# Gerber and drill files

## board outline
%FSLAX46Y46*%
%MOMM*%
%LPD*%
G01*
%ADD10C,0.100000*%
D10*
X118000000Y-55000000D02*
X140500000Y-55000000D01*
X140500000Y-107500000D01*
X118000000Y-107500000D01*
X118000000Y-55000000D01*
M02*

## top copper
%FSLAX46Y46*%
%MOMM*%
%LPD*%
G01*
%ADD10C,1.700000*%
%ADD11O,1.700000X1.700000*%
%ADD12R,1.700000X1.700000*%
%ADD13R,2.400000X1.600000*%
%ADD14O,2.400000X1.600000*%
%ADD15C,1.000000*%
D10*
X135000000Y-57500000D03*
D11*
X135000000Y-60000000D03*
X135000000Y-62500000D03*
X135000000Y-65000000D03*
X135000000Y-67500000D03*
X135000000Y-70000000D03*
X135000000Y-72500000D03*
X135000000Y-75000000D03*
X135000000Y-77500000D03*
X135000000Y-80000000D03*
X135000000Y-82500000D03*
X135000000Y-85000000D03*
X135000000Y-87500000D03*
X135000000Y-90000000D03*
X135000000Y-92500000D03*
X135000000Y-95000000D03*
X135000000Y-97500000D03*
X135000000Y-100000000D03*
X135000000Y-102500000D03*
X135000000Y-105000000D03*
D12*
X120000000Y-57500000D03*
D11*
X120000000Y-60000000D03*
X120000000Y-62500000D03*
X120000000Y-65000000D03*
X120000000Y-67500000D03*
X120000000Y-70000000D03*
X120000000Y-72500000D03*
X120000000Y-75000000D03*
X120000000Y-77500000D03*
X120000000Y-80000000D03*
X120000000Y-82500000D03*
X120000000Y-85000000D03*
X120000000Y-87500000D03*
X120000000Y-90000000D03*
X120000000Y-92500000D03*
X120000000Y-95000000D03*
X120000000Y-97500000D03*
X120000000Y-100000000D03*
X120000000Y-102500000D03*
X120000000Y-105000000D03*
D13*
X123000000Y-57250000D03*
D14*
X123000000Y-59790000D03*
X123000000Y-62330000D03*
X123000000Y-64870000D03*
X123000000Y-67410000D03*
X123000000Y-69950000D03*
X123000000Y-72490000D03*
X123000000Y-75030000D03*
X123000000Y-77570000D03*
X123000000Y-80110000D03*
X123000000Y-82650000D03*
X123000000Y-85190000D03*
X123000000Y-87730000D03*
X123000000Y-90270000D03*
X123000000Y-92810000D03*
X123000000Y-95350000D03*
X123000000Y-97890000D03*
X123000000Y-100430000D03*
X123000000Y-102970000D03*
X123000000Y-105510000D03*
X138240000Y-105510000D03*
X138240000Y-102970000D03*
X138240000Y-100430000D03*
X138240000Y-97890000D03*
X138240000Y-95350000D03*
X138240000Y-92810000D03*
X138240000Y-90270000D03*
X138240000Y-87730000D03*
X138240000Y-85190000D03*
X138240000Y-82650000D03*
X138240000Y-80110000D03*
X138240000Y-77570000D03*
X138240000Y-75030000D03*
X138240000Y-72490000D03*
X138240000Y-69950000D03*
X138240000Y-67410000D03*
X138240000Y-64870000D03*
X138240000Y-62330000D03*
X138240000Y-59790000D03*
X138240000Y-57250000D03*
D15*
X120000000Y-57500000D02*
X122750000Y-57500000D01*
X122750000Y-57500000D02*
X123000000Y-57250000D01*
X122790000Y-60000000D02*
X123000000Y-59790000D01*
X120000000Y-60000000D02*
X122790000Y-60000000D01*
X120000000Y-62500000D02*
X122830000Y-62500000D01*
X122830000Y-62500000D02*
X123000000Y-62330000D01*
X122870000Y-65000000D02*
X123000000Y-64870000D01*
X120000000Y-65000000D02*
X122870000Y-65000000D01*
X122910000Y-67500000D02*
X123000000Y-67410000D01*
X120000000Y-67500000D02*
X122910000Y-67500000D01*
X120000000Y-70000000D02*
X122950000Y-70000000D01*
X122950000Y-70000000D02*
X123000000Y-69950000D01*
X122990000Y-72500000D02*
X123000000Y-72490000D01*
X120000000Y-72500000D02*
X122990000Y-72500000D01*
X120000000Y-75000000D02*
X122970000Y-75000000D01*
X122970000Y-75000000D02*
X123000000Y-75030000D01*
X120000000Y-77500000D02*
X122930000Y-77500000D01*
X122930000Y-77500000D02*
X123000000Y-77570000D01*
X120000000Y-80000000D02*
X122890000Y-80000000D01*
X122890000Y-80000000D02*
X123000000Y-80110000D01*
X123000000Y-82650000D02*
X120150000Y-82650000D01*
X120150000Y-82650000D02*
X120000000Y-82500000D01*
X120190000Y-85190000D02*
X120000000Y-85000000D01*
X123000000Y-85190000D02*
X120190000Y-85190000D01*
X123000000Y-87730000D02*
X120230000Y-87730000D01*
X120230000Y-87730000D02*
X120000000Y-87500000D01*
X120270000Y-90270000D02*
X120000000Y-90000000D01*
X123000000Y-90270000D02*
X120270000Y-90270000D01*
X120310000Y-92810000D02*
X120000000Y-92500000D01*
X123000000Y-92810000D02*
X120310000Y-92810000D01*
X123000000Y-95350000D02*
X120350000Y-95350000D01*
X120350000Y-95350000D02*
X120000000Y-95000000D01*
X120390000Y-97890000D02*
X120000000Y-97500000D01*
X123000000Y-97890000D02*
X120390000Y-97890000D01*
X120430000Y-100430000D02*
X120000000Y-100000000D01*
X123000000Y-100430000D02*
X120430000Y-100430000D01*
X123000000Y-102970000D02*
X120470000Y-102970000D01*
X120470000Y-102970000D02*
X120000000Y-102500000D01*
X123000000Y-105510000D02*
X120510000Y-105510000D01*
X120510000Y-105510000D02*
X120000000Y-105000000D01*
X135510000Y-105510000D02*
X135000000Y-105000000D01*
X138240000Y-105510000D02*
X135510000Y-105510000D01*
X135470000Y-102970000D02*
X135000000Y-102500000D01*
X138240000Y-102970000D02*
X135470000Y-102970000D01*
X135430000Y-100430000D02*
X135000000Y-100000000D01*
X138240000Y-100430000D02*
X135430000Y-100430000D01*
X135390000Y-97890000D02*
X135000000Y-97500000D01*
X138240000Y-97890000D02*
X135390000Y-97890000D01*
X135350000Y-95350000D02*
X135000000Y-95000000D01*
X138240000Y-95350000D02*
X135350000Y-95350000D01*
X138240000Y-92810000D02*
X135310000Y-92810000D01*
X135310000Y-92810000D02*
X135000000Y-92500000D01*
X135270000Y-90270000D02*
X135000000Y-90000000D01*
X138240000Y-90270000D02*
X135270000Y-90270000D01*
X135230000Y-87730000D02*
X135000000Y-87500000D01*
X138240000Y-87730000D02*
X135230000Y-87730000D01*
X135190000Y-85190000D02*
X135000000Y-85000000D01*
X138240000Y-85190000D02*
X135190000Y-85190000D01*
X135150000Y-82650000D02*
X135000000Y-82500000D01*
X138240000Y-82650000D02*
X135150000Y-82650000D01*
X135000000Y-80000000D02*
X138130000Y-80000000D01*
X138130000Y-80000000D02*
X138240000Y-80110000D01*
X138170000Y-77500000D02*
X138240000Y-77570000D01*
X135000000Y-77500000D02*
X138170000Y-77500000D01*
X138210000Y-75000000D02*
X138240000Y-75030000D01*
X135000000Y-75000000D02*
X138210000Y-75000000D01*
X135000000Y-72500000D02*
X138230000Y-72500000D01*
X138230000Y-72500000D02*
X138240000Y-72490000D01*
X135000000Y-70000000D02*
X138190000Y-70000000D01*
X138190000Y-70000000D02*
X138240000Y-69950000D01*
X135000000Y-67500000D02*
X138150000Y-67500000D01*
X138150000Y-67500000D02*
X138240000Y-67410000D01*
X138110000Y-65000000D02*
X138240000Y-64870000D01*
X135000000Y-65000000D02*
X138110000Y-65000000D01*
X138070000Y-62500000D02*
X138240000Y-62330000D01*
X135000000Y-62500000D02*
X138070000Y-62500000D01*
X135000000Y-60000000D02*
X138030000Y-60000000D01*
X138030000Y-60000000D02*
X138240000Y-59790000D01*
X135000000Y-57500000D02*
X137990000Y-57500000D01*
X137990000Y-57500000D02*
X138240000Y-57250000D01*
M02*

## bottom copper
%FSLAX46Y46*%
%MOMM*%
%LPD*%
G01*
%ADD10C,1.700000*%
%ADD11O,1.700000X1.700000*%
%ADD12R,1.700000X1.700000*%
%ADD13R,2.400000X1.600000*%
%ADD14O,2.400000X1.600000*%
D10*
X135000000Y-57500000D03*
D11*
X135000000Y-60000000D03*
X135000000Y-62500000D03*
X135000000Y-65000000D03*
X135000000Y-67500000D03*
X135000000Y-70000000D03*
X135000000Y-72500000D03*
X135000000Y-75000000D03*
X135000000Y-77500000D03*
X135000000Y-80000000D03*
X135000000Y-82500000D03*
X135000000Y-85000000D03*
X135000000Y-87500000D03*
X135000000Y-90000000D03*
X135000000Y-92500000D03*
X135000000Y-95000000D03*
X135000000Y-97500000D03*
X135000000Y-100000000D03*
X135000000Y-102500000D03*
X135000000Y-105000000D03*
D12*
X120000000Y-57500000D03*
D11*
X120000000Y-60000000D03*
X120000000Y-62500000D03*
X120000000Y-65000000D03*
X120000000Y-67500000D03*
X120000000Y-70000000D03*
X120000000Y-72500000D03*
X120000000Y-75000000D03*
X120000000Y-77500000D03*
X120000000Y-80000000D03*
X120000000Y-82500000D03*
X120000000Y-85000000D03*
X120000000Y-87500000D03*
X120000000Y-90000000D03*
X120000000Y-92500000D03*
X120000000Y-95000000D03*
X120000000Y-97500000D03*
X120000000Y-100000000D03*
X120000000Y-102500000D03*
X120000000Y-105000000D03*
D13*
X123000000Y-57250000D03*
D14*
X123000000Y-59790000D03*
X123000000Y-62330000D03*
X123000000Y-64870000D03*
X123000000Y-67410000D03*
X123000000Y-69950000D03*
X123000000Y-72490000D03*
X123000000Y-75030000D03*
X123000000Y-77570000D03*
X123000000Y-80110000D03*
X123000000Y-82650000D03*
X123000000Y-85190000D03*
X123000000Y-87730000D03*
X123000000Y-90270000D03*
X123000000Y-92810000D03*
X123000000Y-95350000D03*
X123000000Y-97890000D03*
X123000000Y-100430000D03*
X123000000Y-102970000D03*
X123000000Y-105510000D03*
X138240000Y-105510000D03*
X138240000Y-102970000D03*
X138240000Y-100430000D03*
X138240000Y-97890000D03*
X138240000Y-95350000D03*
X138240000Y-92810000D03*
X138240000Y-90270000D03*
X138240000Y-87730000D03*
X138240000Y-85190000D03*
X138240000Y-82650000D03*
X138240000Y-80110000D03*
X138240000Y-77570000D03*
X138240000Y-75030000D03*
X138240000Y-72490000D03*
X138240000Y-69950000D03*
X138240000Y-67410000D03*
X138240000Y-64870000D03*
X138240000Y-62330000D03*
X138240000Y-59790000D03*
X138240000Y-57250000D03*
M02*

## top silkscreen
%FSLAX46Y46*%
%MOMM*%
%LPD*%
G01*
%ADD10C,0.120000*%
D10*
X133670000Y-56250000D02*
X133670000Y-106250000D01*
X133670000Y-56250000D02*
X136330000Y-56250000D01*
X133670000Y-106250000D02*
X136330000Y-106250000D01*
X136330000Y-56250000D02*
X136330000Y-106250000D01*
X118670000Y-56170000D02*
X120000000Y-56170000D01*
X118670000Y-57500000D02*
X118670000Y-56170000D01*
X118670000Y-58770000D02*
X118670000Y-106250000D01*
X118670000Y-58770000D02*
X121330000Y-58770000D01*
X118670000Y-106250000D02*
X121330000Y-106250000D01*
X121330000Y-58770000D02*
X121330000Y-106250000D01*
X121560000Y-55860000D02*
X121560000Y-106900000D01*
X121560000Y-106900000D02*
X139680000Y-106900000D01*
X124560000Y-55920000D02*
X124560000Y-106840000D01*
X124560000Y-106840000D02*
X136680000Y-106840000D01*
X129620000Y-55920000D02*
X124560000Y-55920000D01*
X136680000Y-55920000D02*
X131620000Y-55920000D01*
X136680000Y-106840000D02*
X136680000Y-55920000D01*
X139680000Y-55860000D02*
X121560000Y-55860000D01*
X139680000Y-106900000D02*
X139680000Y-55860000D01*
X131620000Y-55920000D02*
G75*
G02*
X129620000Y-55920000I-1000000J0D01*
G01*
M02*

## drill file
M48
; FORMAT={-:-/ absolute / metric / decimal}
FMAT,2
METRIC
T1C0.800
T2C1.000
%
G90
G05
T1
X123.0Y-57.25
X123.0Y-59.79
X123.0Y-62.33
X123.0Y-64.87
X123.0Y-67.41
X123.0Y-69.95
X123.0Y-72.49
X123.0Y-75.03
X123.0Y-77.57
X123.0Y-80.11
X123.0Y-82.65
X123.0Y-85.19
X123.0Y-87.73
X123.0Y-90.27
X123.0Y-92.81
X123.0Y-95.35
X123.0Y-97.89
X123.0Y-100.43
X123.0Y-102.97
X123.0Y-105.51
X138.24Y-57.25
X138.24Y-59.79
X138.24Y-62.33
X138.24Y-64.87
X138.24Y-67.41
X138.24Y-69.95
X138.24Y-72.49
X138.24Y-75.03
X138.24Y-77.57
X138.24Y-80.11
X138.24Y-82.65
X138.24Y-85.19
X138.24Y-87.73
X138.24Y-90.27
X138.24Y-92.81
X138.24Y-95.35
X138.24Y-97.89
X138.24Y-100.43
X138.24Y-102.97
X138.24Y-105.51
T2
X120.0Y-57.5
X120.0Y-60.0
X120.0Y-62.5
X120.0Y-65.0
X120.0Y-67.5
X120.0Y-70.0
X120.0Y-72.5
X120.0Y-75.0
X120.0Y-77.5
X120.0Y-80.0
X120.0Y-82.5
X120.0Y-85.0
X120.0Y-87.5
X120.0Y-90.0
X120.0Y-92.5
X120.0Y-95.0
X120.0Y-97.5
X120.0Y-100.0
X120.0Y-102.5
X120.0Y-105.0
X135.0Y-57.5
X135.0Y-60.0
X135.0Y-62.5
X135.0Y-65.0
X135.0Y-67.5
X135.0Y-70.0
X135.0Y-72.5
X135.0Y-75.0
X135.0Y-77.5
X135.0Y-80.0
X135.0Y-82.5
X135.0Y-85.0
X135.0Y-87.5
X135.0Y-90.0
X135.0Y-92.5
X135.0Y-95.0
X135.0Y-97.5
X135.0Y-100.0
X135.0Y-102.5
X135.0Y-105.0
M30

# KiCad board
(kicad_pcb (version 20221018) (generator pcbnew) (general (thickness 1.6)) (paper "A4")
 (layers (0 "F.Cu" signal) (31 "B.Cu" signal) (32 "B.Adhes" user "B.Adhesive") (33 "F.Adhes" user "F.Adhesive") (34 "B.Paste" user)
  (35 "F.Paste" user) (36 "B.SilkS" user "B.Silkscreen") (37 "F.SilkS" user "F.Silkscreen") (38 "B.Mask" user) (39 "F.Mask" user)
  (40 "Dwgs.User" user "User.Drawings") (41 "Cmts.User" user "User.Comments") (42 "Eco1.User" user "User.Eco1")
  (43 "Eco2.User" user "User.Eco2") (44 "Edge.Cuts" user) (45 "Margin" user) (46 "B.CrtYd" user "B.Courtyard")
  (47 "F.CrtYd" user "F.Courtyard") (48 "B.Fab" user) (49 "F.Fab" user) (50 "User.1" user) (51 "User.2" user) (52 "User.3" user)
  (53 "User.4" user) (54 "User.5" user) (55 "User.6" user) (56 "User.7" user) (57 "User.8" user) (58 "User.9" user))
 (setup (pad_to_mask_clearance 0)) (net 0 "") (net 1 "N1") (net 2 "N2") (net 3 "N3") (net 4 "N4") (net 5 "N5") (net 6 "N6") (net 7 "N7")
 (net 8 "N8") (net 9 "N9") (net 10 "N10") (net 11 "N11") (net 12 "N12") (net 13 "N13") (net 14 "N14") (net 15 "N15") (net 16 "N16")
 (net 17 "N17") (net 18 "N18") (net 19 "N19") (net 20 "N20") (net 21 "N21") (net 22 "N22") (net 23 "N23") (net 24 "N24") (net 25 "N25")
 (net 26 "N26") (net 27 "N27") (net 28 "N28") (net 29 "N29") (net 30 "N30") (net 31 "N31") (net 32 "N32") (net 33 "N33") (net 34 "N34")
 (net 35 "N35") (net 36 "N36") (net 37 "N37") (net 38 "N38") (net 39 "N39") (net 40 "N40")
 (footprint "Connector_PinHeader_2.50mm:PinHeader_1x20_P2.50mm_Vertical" (layer "F.Cu") (at 135 60)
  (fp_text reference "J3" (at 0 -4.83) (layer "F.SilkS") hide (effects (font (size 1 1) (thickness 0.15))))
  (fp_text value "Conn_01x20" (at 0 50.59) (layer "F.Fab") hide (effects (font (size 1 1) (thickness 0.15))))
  (fp_line (start -1.33 -3.75) (end -1.33 46.25) (stroke (width 0.12) (type solid)) (layer "F.SilkS"))
  (fp_line (start -1.33 -3.75) (end 1.33 -3.75) (stroke (width 0.12) (type solid)) (layer "F.SilkS"))
  (fp_line (start -1.33 46.25) (end 1.33 46.25) (stroke (width 0.12) (type solid)) (layer "F.SilkS"))
  (fp_line (start 1.33 -3.75) (end 1.33 46.25) (stroke (width 0.12) (type solid)) (layer "F.SilkS"))
  (pad "1" thru_hole circle (at 0 -2.5) (size 1.7 1.7) (drill 1) (layers "*.Cu" "*.Mask") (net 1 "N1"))
  (pad "2" thru_hole oval (at 0 0) (size 1.7 1.7) (drill 1) (layers "*.Cu" "*.Mask") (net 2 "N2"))
  (pad "3" thru_hole oval (at 0 2.5) (size 1.7 1.7) (drill 1) (layers "*.Cu" "*.Mask") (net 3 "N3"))
  (pad "4" thru_hole oval (at 0 5) (size 1.7 1.7) (drill 1) (layers "*.Cu" "*.Mask") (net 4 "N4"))
  (pad "5" thru_hole oval (at 0 7.5) (size 1.7 1.7) (drill 1) (layers "*.Cu" "*.Mask") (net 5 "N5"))
  (pad "6" thru_hole oval (at 0 10) (size 1.7 1.7) (drill 1) (layers "*.Cu" "*.Mask") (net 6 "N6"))
  (pad "7" thru_hole oval (at 0 12.5) (size 1.7 1.7) (drill 1) (layers "*.Cu" "*.Mask") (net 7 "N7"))
  (pad "8" thru_hole oval (at 0 15) (size 1.7 1.7) (drill 1) (layers "*.Cu" "*.Mask") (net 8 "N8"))
  (pad "9" thru_hole oval (at 0 17.5) (size 1.7 1.7) (drill 1) (layers "*.Cu" "*.Mask") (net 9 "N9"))
  (pad "10" thru_hole oval (at 0 20) (size 1.7 1.7) (drill 1) (layers "*.Cu" "*.Mask") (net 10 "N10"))
  (pad "11" thru_hole oval (at 0 22.5) (size 1.7 1.7) (drill 1) (layers "*.Cu" "*.Mask") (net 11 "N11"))
  (pad "12" thru_hole oval (at 0 25) (size 1.7 1.7) (drill 1) (layers "*.Cu" "*.Mask") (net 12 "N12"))
  (pad "13" thru_hole oval (at 0 27.5) (size 1.7 1.7) (drill 1) (layers "*.Cu" "*.Mask") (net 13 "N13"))
  (pad "14" thru_hole oval (at 0 30) (size 1.7 1.7) (drill 1) (layers "*.Cu" "*.Mask") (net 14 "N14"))
  (pad "15" thru_hole oval (at 0 32.5) (size 1.7 1.7) (drill 1) (layers "*.Cu" "*.Mask") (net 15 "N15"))
  (pad "16" thru_hole oval (at 0 35) (size 1.7 1.7) (drill 1) (layers "*.Cu" "*.Mask") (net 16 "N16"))
  (pad "17" thru_hole oval (at 0 37.5) (size 1.7 1.7) (drill 1) (layers "*.Cu" "*.Mask") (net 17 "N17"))
  (pad "18" thru_hole oval (at 0 40) (size 1.7 1.7) (drill 1) (layers "*.Cu" "*.Mask") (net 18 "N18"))
  (pad "19" thru_hole oval (at 0 42.5) (size 1.7 1.7) (drill 1) (layers "*.Cu" "*.Mask") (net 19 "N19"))
  (pad "20" thru_hole oval (at 0 45) (size 1.7 1.7) (drill 1) (layers "*.Cu" "*.Mask") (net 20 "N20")))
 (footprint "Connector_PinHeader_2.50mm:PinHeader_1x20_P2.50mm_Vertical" (layer "F.Cu") (at 120 60)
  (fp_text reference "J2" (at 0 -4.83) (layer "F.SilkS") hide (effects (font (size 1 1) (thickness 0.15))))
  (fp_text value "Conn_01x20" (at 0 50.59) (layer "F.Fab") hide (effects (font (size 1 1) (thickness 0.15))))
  (fp_line (start -1.33 -3.83) (end 0 -3.83) (stroke (width 0.12) (type solid)) (layer "F.SilkS"))
  (fp_line (start -1.33 -2.5) (end -1.33 -3.83) (stroke (width 0.12) (type solid)) (layer "F.SilkS"))
  (fp_line (start -1.33 -1.23) (end -1.33 46.25) (stroke (width 0.12) (type solid)) (layer "F.SilkS"))
  (fp_line (start -1.33 -1.23) (end 1.33 -1.23) (stroke (width 0.12) (type solid)) (layer "F.SilkS"))
  (fp_line (start -1.33 46.25) (end 1.33 46.25) (stroke (width 0.12) (type solid)) (layer "F.SilkS"))
  (fp_line (start 1.33 -1.23) (end 1.33 46.25) (stroke (width 0.12) (type solid)) (layer "F.SilkS"))
  (pad "1" thru_hole rect (at 0 -2.5) (size 1.7 1.7) (drill 1) (layers "*.Cu" "*.Mask") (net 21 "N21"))
  (pad "2" thru_hole oval (at 0 0) (size 1.7 1.7) (drill 1) (layers "*.Cu" "*.Mask") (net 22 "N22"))
  (pad "3" thru_hole oval (at 0 2.5) (size 1.7 1.7) (drill 1) (layers "*.Cu" "*.Mask") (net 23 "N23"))
  (pad "4" thru_hole oval (at 0 5) (size 1.7 1.7) (drill 1) (layers "*.Cu" "*.Mask") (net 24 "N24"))
  (pad "5" thru_hole oval (at 0 7.5) (size 1.7 1.7) (drill 1) (layers "*.Cu" "*.Mask") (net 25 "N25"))
  (pad "6" thru_hole oval (at 0 10) (size 1.7 1.7) (drill 1) (layers "*.Cu" "*.Mask") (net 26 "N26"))
  (pad "7" thru_hole oval (at 0 12.5) (size 1.7 1.7) (drill 1) (layers "*.Cu" "*.Mask") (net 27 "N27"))
  (pad "8" thru_hole oval (at 0 15) (size 1.7 1.7) (drill 1) (layers "*.Cu" "*.Mask") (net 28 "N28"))
  (pad "9" thru_hole oval (at 0 17.5) (size 1.7 1.7) (drill 1) (layers "*.Cu" "*.Mask") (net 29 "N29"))
  (pad "10" thru_hole oval (at 0 20) (size 1.7 1.7) (drill 1) (layers "*.Cu" "*.Mask") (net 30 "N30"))
  (pad "11" thru_hole oval (at 0 22.5) (size 1.7 1.7) (drill 1) (layers "*.Cu" "*.Mask") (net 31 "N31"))
  (pad "12" thru_hole oval (at 0 25) (size 1.7 1.7) (drill 1) (layers "*.Cu" "*.Mask") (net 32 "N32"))
  (pad "13" thru_hole oval (at 0 27.5) (size 1.7 1.7) (drill 1) (layers "*.Cu" "*.Mask") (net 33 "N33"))
  (pad "14" thru_hole oval (at 0 30) (size 1.7 1.7) (drill 1) (layers "*.Cu" "*.Mask") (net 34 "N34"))
  (pad "15" thru_hole oval (at 0 32.5) (size 1.7 1.7) (drill 1) (layers "*.Cu" "*.Mask") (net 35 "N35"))
  (pad "16" thru_hole oval (at 0 35) (size 1.7 1.7) (drill 1) (layers "*.Cu" "*.Mask") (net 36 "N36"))
  (pad "17" thru_hole oval (at 0 37.5) (size 1.7 1.7) (drill 1) (layers "*.Cu" "*.Mask") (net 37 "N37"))
  (pad "18" thru_hole oval (at 0 40) (size 1.7 1.7) (drill 1) (layers "*.Cu" "*.Mask") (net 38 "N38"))
  (pad "19" thru_hole oval (at 0 42.5) (size 1.7 1.7) (drill 1) (layers "*.Cu" "*.Mask") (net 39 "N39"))
  (pad "20" thru_hole oval (at 0 45) (size 1.7 1.7) (drill 1) (layers "*.Cu" "*.Mask") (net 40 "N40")))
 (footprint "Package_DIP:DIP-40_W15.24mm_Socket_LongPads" (layer "F.Cu") (at 123 57.25)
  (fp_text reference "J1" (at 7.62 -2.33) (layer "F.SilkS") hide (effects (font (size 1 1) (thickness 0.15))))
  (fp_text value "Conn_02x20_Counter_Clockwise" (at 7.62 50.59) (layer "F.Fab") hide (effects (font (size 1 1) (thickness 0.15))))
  (fp_line (start -1.44 -1.39) (end -1.44 49.65) (stroke (width 0.12) (type solid)) (layer "F.SilkS"))
  (fp_line (start -1.44 49.65) (end 16.68 49.65) (stroke (width 0.12) (type solid)) (layer "F.SilkS"))
  (fp_line (start 1.56 -1.33) (end 1.56 49.59) (stroke (width 0.12) (type solid)) (layer "F.SilkS"))
  (fp_line (start 1.56 49.59) (end 13.68 49.59) (stroke (width 0.12) (type solid)) (layer "F.SilkS"))
  (fp_line (start 6.62 -1.33) (end 1.56 -1.33) (stroke (width 0.12) (type solid)) (layer "F.SilkS"))
  (fp_line (start 13.68 -1.33) (end 8.62 -1.33) (stroke (width 0.12) (type solid)) (layer "F.SilkS"))
  (fp_line (start 13.68 49.59) (end 13.68 -1.33) (stroke (width 0.12) (type solid)) (layer "F.SilkS"))
  (fp_line (start 16.68 -1.39) (end -1.44 -1.39) (stroke (width 0.12) (type solid)) (layer "F.SilkS"))
  (fp_line (start 16.68 49.65) (end 16.68 -1.39) (stroke (width 0.12) (type solid)) (layer "F.SilkS"))
  (fp_arc (start 8.62 -1.33) (mid 7.62 -0.33) (end 6.62 -1.33) (stroke (width 0.12) (type solid)) (layer "F.SilkS"))
  (pad "1" thru_hole rect (at 0 0) (size 2.4 1.6) (drill 0.8) (layers "*.Cu" "*.Mask") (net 21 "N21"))
  (pad "2" thru_hole oval (at 0 2.54) (size 2.4 1.6) (drill 0.8) (layers "*.Cu" "*.Mask") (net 22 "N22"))
  (pad "3" thru_hole oval (at 0 5.08) (size 2.4 1.6) (drill 0.8) (layers "*.Cu" "*.Mask") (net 23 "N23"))
  (pad "4" thru_hole oval (at 0 7.62) (size 2.4 1.6) (drill 0.8) (layers "*.Cu" "*.Mask") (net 24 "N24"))
  (pad "5" thru_hole oval (at 0 10.16) (size 2.4 1.6) (drill 0.8) (layers "*.Cu" "*.Mask") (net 25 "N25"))
  (pad "6" thru_hole oval (at 0 12.7) (size 2.4 1.6) (drill 0.8) (layers "*.Cu" "*.Mask") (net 26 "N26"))
  (pad "7" thru_hole oval (at 0 15.24) (size 2.4 1.6) (drill 0.8) (layers "*.Cu" "*.Mask") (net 27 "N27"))
  (pad "8" thru_hole oval (at 0 17.78) (size 2.4 1.6) (drill 0.8) (layers "*.Cu" "*.Mask") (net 28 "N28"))
  (pad "9" thru_hole oval (at 0 20.32) (size 2.4 1.6) (drill 0.8) (layers "*.Cu" "*.Mask") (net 29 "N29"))
  (pad "10" thru_hole oval (at 0 22.86) (size 2.4 1.6) (drill 0.8) (layers "*.Cu" "*.Mask") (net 30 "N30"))
  (pad "11" thru_hole oval (at 0 25.4) (size 2.4 1.6) (drill 0.8) (layers "*.Cu" "*.Mask") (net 31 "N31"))
  (pad "12" thru_hole oval (at 0 27.94) (size 2.4 1.6) (drill 0.8) (layers "*.Cu" "*.Mask") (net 32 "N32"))
  (pad "13" thru_hole oval (at 0 30.48) (size 2.4 1.6) (drill 0.8) (layers "*.Cu" "*.Mask") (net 33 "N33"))
  (pad "14" thru_hole oval (at 0 33.02) (size 2.4 1.6) (drill 0.8) (layers "*.Cu" "*.Mask") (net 34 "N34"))
  (pad "15" thru_hole oval (at 0 35.56) (size 2.4 1.6) (drill 0.8) (layers "*.Cu" "*.Mask") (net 35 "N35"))
  (pad "16" thru_hole oval (at 0 38.1) (size 2.4 1.6) (drill 0.8) (layers "*.Cu" "*.Mask") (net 36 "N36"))
  (pad "17" thru_hole oval (at 0 40.64) (size 2.4 1.6) (drill 0.8) (layers "*.Cu" "*.Mask") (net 37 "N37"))
  (pad "18" thru_hole oval (at 0 43.18) (size 2.4 1.6) (drill 0.8) (layers "*.Cu" "*.Mask") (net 38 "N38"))
  (pad "19" thru_hole oval (at 0 45.72) (size 2.4 1.6) (drill 0.8) (layers "*.Cu" "*.Mask") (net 39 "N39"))
  (pad "20" thru_hole oval (at 0 48.26) (size 2.4 1.6) (drill 0.8) (layers "*.Cu" "*.Mask") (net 40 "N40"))
  (pad "21" thru_hole oval (at 15.24 48.26) (size 2.4 1.6) (drill 0.8) (layers "*.Cu" "*.Mask") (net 20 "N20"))
  (pad "22" thru_hole oval (at 15.24 45.72) (size 2.4 1.6) (drill 0.8) (layers "*.Cu" "*.Mask") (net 19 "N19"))
  (pad "23" thru_hole oval (at 15.24 43.18) (size 2.4 1.6) (drill 0.8) (layers "*.Cu" "*.Mask") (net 18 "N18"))
  (pad "24" thru_hole oval (at 15.24 40.64) (size 2.4 1.6) (drill 0.8) (layers "*.Cu" "*.Mask") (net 17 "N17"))
  (pad "25" thru_hole oval (at 15.24 38.1) (size 2.4 1.6) (drill 0.8) (layers "*.Cu" "*.Mask") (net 16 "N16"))
  (pad "26" thru_hole oval (at 15.24 35.56) (size 2.4 1.6) (drill 0.8) (layers "*.Cu" "*.Mask") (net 15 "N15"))
  (pad "27" thru_hole oval (at 15.24 33.02) (size 2.4 1.6) (drill 0.8) (layers "*.Cu" "*.Mask") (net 14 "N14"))
  (pad "28" thru_hole oval (at 15.24 30.48) (size 2.4 1.6) (drill 0.8) (layers "*.Cu" "*.Mask") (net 13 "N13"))
  (pad "29" thru_hole oval (at 15.24 27.94) (size 2.4 1.6) (drill 0.8) (layers "*.Cu" "*.Mask") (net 12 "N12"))
  (pad "30" thru_hole oval (at 15.24 25.4) (size 2.4 1.6) (drill 0.8) (layers "*.Cu" "*.Mask") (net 11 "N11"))
  (pad "31" thru_hole oval (at 15.24 22.86) (size 2.4 1.6) (drill 0.8) (layers "*.Cu" "*.Mask") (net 10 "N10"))
  (pad "32" thru_hole oval (at 15.24 20.32) (size 2.4 1.6) (drill 0.8) (layers "*.Cu" "*.Mask") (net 9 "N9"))
  (pad "33" thru_hole oval (at 15.24 17.78) (size 2.4 1.6) (drill 0.8) (layers "*.Cu" "*.Mask") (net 8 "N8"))
  (pad "34" thru_hole oval (at 15.24 15.24) (size 2.4 1.6) (drill 0.8) (layers "*.Cu" "*.Mask") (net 7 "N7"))
  (pad "35" thru_hole oval (at 15.24 12.7) (size 2.4 1.6) (drill 0.8) (layers "*.Cu" "*.Mask") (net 6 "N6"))
  (pad "36" thru_hole oval (at 15.24 10.16) (size 2.4 1.6) (drill 0.8) (layers "*.Cu" "*.Mask") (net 5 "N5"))
  (pad "37" thru_hole oval (at 15.24 7.62) (size 2.4 1.6) (drill 0.8) (layers "*.Cu" "*.Mask") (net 4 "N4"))
  (pad "38" thru_hole oval (at 15.24 5.08) (size 2.4 1.6) (drill 0.8) (layers "*.Cu" "*.Mask") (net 3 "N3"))
  (pad "39" thru_hole oval (at 15.24 2.54) (size 2.4 1.6) (drill 0.8) (layers "*.Cu" "*.Mask") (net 2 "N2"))
  (pad "40" thru_hole oval (at 15.24 0) (size 2.4 1.6) (drill 0.8) (layers "*.Cu" "*.Mask") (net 1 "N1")))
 (gr_rect (start 118 55) (end 140.5 107.5) (stroke (width 0.1) (type default)) (fill none) (layer "Edge.Cuts"))
 (segment (start 120 57.5) (end 122.75 57.5) (width 1) (layer "F.Cu") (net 21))
 (segment (start 122.75 57.5) (end 123 57.25) (width 1) (layer "F.Cu") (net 21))
 (segment (start 122.79 60) (end 123 59.79) (width 1) (layer "F.Cu") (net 22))
 (segment (start 120 60) (end 122.79 60) (width 1) (layer "F.Cu") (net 22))
 (segment (start 120 62.5) (end 122.83 62.5) (width 1) (layer "F.Cu") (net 23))
 (segment (start 122.83 62.5) (end 123 62.33) (width 1) (layer "F.Cu") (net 23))
 (segment (start 122.87 65) (end 123 64.87) (width 1) (layer "F.Cu") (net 24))
 (segment (start 120 65) (end 122.87 65) (width 1) (layer "F.Cu") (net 24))
 (segment (start 122.91 67.5) (end 123 67.41) (width 1) (layer "F.Cu") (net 25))
 (segment (start 120 67.5) (end 122.91 67.5) (width 1) (layer "F.Cu") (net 25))
 (segment (start 120 70) (end 122.95 70) (width 1) (layer "F.Cu") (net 26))
 (segment (start 122.95 70) (end 123 69.95) (width 1) (layer "F.Cu") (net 26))
 (segment (start 122.99 72.5) (end 123 72.49) (width 1) (layer "F.Cu") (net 27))
 (segment (start 120 72.5) (end 122.99 72.5) (width 1) (layer "F.Cu") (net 27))
 (segment (start 120 75) (end 122.97 75) (width 1) (layer "F.Cu") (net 28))
 (segment (start 122.97 75) (end 123 75.03) (width 1) (layer "F.Cu") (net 28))
 (segment (start 120 77.5) (end 122.93 77.5) (width 1) (layer "F.Cu") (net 29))
 (segment (start 122.93 77.5) (end 123 77.57) (width 1) (layer "F.Cu") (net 29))
 (segment (start 120 80) (end 122.89 80) (width 1) (layer "F.Cu") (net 30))
 (segment (start 122.89 80) (end 123 80.11) (width 1) (layer "F.Cu") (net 30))
 (segment (start 123 82.65) (end 120.15 82.65) (width 1) (layer "F.Cu") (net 31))
 (segment (start 120.15 82.65) (end 120 82.5) (width 1) (layer "F.Cu") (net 31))
 (segment (start 120.19 85.19) (end 120 85) (width 1) (layer "F.Cu") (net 32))
 (segment (start 123 85.19) (end 120.19 85.19) (width 1) (layer "F.Cu") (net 32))
 (segment (start 123 87.73) (end 120.23 87.73) (width 1) (layer "F.Cu") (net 33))
 (segment (start 120.23 87.73) (end 120 87.5) (width 1) (layer "F.Cu") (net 33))
 (segment (start 120.27 90.27) (end 120 90) (width 1) (layer "F.Cu") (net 34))
 (segment (start 123 90.27) (end 120.27 90.27) (width 1) (layer "F.Cu") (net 34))
 (segment (start 120.31 92.81) (end 120 92.5) (width 1) (layer "F.Cu") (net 35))
 (segment (start 123 92.81) (end 120.31 92.81) (width 1) (layer "F.Cu") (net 35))
 (segment (start 123 95.35) (end 120.35 95.35) (width 1) (layer "F.Cu") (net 36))
 (segment (start 120.35 95.35) (end 120 95) (width 1) (layer "F.Cu") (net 36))
 (segment (start 120.39 97.89) (end 120 97.5) (width 1) (layer "F.Cu") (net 37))
 (segment (start 123 97.89) (end 120.39 97.89) (width 1) (layer "F.Cu") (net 37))
 (segment (start 120.43 100.43) (end 120 100) (width 1) (layer "F.Cu") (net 38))
 (segment (start 123 100.43) (end 120.43 100.43) (width 1) (layer "F.Cu") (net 38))
 (segment (start 123 102.97) (end 120.47 102.97) (width 1) (layer "F.Cu") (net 39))
 (segment (start 120.47 102.97) (end 120 102.5) (width 1) (layer "F.Cu") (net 39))
 (segment (start 123 105.51) (end 120.51 105.51) (width 1) (layer "F.Cu") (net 40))
 (segment (start 120.51 105.51) (end 120 105) (width 1) (layer "F.Cu") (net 40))
 (segment (start 135.51 105.51) (end 135 105) (width 1) (layer "F.Cu") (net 20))
 (segment (start 138.24 105.51) (end 135.51 105.51) (width 1) (layer "F.Cu") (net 20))
 (segment (start 135.47 102.97) (end 135 102.5) (width 1) (layer "F.Cu") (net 19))
 (segment (start 138.24 102.97) (end 135.47 102.97) (width 1) (layer "F.Cu") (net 19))
 (segment (start 135.43 100.43) (end 135 100) (width 1) (layer "F.Cu") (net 18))
 (segment (start 138.24 100.43) (end 135.43 100.43) (width 1) (layer "F.Cu") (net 18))
 (segment (start 135.39 97.89) (end 135 97.5) (width 1) (layer "F.Cu") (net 17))
 (segment (start 138.24 97.89) (end 135.39 97.89) (width 1) (layer "F.Cu") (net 17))
 (segment (start 135.35 95.35) (end 135 95) (width 1) (layer "F.Cu") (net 16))
 (segment (start 138.24 95.35) (end 135.35 95.35) (width 1) (layer "F.Cu") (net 16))
 (segment (start 138.24 92.81) (end 135.31 92.81) (width 1) (layer "F.Cu") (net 15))
 (segment (start 135.31 92.81) (end 135 92.5) (width 1) (layer "F.Cu") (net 15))
 (segment (start 135.27 90.27) (end 135 90) (width 1) (layer "F.Cu") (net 14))
 (segment (start 138.24 90.27) (end 135.27 90.27) (width 1) (layer "F.Cu") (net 14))
 (segment (start 135.23 87.73) (end 135 87.5) (width 1) (layer "F.Cu") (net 13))
 (segment (start 138.24 87.73) (end 135.23 87.73) (width 1) (layer "F.Cu") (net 13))
 (segment (start 135.19 85.19) (end 135 85) (width 1) (layer "F.Cu") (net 12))
 (segment (start 138.24 85.19) (end 135.19 85.19) (width 1) (layer "F.Cu") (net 12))
 (segment (start 135.15 82.65) (end 135 82.5) (width 1) (layer "F.Cu") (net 11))
 (segment (start 138.24 82.65) (end 135.15 82.65) (width 1) (layer "F.Cu") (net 11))
 (segment (start 135 80) (end 138.13 80) (width 1) (layer "F.Cu") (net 10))
 (segment (start 138.13 80) (end 138.24 80.11) (width 1) (layer "F.Cu") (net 10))
 (segment (start 138.17 77.5) (end 138.24 77.57) (width 1) (layer "F.Cu") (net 9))
 (segment (start 135 77.5) (end 138.17 77.5) (width 1) (layer "F.Cu") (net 9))
 (segment (start 138.21 75) (end 138.24 75.03) (width 1) (layer "F.Cu") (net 8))
 (segment (start 135 75) (end 138.21 75) (width 1) (layer "F.Cu") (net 8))
 (segment (start 135 72.5) (end 138.23 72.5) (width 1) (layer "F.Cu") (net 7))
 (segment (start 138.23 72.5) (end 138.24 72.49) (width 1) (layer "F.Cu") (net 7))
 (segment (start 135 70) (end 138.19 70) (width 1) (layer "F.Cu") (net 6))
 (segment (start 138.19 70) (end 138.24 69.95) (width 1) (layer "F.Cu") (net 6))
 (segment (start 135 67.5) (end 138.15 67.5) (width 1) (layer "F.Cu") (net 5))
 (segment (start 138.15 67.5) (end 138.24 67.41) (width 1) (layer "F.Cu") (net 5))
 (segment (start 138.11 65) (end 138.24 64.87) (width 1) (layer "F.Cu") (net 4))
 (segment (start 135 65) (end 138.11 65) (width 1) (layer "F.Cu") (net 4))
 (segment (start 138.07 62.5) (end 138.24 62.33) (width 1) (layer "F.Cu") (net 3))
 (segment (start 135 62.5) (end 138.07 62.5) (width 1) (layer "F.Cu") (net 3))
 (segment (start 135 60) (end 138.03 60) (width 1) (layer "F.Cu") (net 2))
 (segment (start 138.03 60) (end 138.24 59.79) (width 1) (layer "F.Cu") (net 2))
 (segment (start 135 57.5) (end 137.99 57.5) (width 1) (layer "F.Cu") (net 1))
 (segment (start 137.99 57.5) (end 138.24 57.25) (width 1) (layer "F.Cu") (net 1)))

